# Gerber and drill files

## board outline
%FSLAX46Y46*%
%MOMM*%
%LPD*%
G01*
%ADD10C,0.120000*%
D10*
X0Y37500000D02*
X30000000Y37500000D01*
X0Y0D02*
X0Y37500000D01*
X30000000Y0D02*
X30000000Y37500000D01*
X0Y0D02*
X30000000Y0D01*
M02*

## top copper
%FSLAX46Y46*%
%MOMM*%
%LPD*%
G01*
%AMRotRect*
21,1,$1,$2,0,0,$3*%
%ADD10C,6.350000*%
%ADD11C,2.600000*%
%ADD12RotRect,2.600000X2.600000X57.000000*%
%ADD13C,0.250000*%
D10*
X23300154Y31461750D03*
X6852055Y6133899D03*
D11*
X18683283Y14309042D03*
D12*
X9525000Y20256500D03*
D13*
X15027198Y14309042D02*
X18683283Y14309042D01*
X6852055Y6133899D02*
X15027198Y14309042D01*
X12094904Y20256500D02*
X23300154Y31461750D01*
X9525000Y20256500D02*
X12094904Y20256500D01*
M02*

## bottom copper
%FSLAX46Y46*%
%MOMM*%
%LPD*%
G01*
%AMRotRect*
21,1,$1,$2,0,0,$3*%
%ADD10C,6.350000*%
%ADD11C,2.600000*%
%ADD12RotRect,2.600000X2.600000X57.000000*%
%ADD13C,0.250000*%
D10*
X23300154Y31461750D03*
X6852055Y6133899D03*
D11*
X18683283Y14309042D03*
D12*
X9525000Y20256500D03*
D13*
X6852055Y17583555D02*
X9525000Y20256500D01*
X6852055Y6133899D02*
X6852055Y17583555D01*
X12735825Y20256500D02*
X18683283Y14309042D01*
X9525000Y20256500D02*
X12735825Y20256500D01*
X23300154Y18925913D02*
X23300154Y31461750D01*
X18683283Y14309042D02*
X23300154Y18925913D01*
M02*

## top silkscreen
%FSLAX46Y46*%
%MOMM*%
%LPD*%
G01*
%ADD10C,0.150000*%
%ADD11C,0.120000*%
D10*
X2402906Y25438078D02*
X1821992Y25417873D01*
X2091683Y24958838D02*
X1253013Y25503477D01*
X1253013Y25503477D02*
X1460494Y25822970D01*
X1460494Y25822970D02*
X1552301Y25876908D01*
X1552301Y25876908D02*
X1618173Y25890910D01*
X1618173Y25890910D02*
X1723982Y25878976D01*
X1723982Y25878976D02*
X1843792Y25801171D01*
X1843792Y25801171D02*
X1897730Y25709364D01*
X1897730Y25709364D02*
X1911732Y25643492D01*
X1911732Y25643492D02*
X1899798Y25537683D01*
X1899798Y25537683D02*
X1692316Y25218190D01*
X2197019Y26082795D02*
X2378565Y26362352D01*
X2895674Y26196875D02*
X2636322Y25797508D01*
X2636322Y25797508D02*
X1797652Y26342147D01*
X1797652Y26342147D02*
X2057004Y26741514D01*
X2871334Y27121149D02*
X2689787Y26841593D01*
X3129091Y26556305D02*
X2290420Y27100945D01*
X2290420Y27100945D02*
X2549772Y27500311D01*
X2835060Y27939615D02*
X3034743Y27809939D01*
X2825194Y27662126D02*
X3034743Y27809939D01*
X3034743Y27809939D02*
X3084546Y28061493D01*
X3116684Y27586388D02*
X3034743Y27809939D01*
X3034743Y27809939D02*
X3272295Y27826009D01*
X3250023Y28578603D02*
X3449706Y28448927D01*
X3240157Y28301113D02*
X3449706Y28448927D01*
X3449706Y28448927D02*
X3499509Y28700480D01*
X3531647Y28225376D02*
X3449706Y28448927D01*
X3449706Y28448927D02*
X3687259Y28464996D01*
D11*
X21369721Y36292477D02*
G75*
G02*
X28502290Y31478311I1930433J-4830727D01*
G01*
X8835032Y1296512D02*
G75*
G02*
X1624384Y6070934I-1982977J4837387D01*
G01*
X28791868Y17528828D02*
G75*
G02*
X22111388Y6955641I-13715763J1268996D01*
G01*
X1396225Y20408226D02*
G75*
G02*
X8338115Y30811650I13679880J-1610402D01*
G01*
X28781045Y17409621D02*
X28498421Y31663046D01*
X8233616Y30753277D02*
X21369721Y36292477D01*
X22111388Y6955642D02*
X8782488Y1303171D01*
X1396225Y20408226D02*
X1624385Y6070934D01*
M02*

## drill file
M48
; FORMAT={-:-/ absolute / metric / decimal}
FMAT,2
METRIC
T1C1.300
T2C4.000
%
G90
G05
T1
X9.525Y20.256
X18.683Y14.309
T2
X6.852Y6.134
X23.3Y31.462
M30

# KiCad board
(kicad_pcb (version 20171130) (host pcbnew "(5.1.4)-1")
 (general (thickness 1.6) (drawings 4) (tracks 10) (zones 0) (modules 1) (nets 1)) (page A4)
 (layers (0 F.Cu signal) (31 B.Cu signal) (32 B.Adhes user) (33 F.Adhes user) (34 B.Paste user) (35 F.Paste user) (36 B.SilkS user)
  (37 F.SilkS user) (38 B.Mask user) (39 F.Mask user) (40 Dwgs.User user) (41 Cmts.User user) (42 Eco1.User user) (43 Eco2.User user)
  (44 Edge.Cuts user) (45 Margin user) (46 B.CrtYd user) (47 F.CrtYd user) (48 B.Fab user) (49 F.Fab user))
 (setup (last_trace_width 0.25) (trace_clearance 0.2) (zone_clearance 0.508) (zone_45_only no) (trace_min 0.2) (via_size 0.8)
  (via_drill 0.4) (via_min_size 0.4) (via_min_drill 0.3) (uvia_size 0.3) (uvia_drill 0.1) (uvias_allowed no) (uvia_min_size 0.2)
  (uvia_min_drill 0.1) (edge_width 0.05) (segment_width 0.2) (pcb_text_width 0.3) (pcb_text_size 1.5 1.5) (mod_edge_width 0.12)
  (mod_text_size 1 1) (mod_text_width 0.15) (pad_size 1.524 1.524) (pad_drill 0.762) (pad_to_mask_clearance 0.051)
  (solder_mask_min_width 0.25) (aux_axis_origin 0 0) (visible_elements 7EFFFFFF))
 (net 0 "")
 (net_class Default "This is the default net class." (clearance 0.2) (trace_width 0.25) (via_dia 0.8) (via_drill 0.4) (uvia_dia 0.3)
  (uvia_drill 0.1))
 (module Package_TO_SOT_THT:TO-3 (layer F.Cu) (at 9.525 -20.2565 57)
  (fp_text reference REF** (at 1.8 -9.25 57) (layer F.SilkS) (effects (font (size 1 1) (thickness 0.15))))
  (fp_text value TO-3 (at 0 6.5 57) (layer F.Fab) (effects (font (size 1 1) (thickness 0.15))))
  (fp_arc (start 16.9 5.45) (end 19.9 1.2) (angle 111.6) (layer F.SilkS) (width 0.12))
  (fp_arc (start -13.3 5.45) (end -16.2 1.1) (angle -111.6) (layer F.SilkS) (width 0.12))
  (fp_arc (start 1.8 5.45) (end -4.3 17.8) (angle -54) (layer F.SilkS) (width 0.12))
  (fp_arc (start 1.8 5.45) (end -4.3 -6.9) (angle 54) (layer F.SilkS) (width 0.12))
  (fp_line (start 8.1 17.7) (end 19.9 9.7) (layer F.SilkS) (width 0.12))
  (fp_line (start 8.1 -6.8) (end 19.9 1.2) (layer F.SilkS) (width 0.12))
  (fp_line (start -4.3 17.8) (end -16.3 9.7) (layer F.SilkS) (width 0.12))
  (fp_line (start -4.3 -6.9) (end -16.2 1.1) (layer F.SilkS) (width 0.12))
  (pad 3 thru_hole circle (at 16.9 5.45 57) (size 6.35 6.35) (drill 4) (layers *.Cu *.Mask))
  (pad 3 thru_hole circle (at -13.3 5.45 57) (size 6.35 6.35) (drill 4) (layers *.Cu *.Mask))
  (pad 2 thru_hole circle (at 0 10.92 57) (size 2.6 2.6) (drill 1.3) (layers *.Cu *.Mask))
  (pad 1 thru_hole rect (at 0 0 57) (size 2.6 2.6) (drill 1.3) (layers *.Cu *.Mask)))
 (gr_line (start 0 -37.5) (end 30 -37.5) (layer Edge.Cuts) (width 0.12))
 (gr_line (start 0 0) (end 0 -37.5) (layer Edge.Cuts) (width 0.12))
 (gr_line (start 30 0) (end 30 -37.5) (layer Edge.Cuts) (width 0.12))
 (gr_line (start 0 0) (end 30 0) (layer Edge.Cuts) (width 0.12))
 (segment (start 15.027198 -14.309042) (end 18.683283 -14.309042) (width 0.25) (layer F.Cu) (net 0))
 (segment (start 6.852055 -6.133899) (end 15.027198 -14.309042) (width 0.25) (layer F.Cu) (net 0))
 (segment (start 12.094904 -20.2565) (end 23.300154 -31.46175) (width 0.25) (layer F.Cu) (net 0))
 (segment (start 9.525 -20.2565) (end 12.094904 -20.2565) (width 0.25) (layer F.Cu) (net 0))
 (segment (start 6.852055 -17.583555) (end 9.525 -20.2565) (width 0.25) (layer B.Cu) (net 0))
 (segment (start 6.852055 -6.133899) (end 6.852055 -17.583555) (width 0.25) (layer B.Cu) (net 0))
 (segment (start 12.735825 -20.2565) (end 18.683283 -14.309042) (width 0.25) (layer B.Cu) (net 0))
 (segment (start 9.525 -20.2565) (end 12.735825 -20.2565) (width 0.25) (layer B.Cu) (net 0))
 (segment (start 23.300154 -18.925913) (end 23.300154 -31.46175) (width 0.25) (layer B.Cu) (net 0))
 (segment (start 18.683283 -14.309042) (end 23.300154 -18.925913) (width 0.25) (layer B.Cu) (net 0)))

